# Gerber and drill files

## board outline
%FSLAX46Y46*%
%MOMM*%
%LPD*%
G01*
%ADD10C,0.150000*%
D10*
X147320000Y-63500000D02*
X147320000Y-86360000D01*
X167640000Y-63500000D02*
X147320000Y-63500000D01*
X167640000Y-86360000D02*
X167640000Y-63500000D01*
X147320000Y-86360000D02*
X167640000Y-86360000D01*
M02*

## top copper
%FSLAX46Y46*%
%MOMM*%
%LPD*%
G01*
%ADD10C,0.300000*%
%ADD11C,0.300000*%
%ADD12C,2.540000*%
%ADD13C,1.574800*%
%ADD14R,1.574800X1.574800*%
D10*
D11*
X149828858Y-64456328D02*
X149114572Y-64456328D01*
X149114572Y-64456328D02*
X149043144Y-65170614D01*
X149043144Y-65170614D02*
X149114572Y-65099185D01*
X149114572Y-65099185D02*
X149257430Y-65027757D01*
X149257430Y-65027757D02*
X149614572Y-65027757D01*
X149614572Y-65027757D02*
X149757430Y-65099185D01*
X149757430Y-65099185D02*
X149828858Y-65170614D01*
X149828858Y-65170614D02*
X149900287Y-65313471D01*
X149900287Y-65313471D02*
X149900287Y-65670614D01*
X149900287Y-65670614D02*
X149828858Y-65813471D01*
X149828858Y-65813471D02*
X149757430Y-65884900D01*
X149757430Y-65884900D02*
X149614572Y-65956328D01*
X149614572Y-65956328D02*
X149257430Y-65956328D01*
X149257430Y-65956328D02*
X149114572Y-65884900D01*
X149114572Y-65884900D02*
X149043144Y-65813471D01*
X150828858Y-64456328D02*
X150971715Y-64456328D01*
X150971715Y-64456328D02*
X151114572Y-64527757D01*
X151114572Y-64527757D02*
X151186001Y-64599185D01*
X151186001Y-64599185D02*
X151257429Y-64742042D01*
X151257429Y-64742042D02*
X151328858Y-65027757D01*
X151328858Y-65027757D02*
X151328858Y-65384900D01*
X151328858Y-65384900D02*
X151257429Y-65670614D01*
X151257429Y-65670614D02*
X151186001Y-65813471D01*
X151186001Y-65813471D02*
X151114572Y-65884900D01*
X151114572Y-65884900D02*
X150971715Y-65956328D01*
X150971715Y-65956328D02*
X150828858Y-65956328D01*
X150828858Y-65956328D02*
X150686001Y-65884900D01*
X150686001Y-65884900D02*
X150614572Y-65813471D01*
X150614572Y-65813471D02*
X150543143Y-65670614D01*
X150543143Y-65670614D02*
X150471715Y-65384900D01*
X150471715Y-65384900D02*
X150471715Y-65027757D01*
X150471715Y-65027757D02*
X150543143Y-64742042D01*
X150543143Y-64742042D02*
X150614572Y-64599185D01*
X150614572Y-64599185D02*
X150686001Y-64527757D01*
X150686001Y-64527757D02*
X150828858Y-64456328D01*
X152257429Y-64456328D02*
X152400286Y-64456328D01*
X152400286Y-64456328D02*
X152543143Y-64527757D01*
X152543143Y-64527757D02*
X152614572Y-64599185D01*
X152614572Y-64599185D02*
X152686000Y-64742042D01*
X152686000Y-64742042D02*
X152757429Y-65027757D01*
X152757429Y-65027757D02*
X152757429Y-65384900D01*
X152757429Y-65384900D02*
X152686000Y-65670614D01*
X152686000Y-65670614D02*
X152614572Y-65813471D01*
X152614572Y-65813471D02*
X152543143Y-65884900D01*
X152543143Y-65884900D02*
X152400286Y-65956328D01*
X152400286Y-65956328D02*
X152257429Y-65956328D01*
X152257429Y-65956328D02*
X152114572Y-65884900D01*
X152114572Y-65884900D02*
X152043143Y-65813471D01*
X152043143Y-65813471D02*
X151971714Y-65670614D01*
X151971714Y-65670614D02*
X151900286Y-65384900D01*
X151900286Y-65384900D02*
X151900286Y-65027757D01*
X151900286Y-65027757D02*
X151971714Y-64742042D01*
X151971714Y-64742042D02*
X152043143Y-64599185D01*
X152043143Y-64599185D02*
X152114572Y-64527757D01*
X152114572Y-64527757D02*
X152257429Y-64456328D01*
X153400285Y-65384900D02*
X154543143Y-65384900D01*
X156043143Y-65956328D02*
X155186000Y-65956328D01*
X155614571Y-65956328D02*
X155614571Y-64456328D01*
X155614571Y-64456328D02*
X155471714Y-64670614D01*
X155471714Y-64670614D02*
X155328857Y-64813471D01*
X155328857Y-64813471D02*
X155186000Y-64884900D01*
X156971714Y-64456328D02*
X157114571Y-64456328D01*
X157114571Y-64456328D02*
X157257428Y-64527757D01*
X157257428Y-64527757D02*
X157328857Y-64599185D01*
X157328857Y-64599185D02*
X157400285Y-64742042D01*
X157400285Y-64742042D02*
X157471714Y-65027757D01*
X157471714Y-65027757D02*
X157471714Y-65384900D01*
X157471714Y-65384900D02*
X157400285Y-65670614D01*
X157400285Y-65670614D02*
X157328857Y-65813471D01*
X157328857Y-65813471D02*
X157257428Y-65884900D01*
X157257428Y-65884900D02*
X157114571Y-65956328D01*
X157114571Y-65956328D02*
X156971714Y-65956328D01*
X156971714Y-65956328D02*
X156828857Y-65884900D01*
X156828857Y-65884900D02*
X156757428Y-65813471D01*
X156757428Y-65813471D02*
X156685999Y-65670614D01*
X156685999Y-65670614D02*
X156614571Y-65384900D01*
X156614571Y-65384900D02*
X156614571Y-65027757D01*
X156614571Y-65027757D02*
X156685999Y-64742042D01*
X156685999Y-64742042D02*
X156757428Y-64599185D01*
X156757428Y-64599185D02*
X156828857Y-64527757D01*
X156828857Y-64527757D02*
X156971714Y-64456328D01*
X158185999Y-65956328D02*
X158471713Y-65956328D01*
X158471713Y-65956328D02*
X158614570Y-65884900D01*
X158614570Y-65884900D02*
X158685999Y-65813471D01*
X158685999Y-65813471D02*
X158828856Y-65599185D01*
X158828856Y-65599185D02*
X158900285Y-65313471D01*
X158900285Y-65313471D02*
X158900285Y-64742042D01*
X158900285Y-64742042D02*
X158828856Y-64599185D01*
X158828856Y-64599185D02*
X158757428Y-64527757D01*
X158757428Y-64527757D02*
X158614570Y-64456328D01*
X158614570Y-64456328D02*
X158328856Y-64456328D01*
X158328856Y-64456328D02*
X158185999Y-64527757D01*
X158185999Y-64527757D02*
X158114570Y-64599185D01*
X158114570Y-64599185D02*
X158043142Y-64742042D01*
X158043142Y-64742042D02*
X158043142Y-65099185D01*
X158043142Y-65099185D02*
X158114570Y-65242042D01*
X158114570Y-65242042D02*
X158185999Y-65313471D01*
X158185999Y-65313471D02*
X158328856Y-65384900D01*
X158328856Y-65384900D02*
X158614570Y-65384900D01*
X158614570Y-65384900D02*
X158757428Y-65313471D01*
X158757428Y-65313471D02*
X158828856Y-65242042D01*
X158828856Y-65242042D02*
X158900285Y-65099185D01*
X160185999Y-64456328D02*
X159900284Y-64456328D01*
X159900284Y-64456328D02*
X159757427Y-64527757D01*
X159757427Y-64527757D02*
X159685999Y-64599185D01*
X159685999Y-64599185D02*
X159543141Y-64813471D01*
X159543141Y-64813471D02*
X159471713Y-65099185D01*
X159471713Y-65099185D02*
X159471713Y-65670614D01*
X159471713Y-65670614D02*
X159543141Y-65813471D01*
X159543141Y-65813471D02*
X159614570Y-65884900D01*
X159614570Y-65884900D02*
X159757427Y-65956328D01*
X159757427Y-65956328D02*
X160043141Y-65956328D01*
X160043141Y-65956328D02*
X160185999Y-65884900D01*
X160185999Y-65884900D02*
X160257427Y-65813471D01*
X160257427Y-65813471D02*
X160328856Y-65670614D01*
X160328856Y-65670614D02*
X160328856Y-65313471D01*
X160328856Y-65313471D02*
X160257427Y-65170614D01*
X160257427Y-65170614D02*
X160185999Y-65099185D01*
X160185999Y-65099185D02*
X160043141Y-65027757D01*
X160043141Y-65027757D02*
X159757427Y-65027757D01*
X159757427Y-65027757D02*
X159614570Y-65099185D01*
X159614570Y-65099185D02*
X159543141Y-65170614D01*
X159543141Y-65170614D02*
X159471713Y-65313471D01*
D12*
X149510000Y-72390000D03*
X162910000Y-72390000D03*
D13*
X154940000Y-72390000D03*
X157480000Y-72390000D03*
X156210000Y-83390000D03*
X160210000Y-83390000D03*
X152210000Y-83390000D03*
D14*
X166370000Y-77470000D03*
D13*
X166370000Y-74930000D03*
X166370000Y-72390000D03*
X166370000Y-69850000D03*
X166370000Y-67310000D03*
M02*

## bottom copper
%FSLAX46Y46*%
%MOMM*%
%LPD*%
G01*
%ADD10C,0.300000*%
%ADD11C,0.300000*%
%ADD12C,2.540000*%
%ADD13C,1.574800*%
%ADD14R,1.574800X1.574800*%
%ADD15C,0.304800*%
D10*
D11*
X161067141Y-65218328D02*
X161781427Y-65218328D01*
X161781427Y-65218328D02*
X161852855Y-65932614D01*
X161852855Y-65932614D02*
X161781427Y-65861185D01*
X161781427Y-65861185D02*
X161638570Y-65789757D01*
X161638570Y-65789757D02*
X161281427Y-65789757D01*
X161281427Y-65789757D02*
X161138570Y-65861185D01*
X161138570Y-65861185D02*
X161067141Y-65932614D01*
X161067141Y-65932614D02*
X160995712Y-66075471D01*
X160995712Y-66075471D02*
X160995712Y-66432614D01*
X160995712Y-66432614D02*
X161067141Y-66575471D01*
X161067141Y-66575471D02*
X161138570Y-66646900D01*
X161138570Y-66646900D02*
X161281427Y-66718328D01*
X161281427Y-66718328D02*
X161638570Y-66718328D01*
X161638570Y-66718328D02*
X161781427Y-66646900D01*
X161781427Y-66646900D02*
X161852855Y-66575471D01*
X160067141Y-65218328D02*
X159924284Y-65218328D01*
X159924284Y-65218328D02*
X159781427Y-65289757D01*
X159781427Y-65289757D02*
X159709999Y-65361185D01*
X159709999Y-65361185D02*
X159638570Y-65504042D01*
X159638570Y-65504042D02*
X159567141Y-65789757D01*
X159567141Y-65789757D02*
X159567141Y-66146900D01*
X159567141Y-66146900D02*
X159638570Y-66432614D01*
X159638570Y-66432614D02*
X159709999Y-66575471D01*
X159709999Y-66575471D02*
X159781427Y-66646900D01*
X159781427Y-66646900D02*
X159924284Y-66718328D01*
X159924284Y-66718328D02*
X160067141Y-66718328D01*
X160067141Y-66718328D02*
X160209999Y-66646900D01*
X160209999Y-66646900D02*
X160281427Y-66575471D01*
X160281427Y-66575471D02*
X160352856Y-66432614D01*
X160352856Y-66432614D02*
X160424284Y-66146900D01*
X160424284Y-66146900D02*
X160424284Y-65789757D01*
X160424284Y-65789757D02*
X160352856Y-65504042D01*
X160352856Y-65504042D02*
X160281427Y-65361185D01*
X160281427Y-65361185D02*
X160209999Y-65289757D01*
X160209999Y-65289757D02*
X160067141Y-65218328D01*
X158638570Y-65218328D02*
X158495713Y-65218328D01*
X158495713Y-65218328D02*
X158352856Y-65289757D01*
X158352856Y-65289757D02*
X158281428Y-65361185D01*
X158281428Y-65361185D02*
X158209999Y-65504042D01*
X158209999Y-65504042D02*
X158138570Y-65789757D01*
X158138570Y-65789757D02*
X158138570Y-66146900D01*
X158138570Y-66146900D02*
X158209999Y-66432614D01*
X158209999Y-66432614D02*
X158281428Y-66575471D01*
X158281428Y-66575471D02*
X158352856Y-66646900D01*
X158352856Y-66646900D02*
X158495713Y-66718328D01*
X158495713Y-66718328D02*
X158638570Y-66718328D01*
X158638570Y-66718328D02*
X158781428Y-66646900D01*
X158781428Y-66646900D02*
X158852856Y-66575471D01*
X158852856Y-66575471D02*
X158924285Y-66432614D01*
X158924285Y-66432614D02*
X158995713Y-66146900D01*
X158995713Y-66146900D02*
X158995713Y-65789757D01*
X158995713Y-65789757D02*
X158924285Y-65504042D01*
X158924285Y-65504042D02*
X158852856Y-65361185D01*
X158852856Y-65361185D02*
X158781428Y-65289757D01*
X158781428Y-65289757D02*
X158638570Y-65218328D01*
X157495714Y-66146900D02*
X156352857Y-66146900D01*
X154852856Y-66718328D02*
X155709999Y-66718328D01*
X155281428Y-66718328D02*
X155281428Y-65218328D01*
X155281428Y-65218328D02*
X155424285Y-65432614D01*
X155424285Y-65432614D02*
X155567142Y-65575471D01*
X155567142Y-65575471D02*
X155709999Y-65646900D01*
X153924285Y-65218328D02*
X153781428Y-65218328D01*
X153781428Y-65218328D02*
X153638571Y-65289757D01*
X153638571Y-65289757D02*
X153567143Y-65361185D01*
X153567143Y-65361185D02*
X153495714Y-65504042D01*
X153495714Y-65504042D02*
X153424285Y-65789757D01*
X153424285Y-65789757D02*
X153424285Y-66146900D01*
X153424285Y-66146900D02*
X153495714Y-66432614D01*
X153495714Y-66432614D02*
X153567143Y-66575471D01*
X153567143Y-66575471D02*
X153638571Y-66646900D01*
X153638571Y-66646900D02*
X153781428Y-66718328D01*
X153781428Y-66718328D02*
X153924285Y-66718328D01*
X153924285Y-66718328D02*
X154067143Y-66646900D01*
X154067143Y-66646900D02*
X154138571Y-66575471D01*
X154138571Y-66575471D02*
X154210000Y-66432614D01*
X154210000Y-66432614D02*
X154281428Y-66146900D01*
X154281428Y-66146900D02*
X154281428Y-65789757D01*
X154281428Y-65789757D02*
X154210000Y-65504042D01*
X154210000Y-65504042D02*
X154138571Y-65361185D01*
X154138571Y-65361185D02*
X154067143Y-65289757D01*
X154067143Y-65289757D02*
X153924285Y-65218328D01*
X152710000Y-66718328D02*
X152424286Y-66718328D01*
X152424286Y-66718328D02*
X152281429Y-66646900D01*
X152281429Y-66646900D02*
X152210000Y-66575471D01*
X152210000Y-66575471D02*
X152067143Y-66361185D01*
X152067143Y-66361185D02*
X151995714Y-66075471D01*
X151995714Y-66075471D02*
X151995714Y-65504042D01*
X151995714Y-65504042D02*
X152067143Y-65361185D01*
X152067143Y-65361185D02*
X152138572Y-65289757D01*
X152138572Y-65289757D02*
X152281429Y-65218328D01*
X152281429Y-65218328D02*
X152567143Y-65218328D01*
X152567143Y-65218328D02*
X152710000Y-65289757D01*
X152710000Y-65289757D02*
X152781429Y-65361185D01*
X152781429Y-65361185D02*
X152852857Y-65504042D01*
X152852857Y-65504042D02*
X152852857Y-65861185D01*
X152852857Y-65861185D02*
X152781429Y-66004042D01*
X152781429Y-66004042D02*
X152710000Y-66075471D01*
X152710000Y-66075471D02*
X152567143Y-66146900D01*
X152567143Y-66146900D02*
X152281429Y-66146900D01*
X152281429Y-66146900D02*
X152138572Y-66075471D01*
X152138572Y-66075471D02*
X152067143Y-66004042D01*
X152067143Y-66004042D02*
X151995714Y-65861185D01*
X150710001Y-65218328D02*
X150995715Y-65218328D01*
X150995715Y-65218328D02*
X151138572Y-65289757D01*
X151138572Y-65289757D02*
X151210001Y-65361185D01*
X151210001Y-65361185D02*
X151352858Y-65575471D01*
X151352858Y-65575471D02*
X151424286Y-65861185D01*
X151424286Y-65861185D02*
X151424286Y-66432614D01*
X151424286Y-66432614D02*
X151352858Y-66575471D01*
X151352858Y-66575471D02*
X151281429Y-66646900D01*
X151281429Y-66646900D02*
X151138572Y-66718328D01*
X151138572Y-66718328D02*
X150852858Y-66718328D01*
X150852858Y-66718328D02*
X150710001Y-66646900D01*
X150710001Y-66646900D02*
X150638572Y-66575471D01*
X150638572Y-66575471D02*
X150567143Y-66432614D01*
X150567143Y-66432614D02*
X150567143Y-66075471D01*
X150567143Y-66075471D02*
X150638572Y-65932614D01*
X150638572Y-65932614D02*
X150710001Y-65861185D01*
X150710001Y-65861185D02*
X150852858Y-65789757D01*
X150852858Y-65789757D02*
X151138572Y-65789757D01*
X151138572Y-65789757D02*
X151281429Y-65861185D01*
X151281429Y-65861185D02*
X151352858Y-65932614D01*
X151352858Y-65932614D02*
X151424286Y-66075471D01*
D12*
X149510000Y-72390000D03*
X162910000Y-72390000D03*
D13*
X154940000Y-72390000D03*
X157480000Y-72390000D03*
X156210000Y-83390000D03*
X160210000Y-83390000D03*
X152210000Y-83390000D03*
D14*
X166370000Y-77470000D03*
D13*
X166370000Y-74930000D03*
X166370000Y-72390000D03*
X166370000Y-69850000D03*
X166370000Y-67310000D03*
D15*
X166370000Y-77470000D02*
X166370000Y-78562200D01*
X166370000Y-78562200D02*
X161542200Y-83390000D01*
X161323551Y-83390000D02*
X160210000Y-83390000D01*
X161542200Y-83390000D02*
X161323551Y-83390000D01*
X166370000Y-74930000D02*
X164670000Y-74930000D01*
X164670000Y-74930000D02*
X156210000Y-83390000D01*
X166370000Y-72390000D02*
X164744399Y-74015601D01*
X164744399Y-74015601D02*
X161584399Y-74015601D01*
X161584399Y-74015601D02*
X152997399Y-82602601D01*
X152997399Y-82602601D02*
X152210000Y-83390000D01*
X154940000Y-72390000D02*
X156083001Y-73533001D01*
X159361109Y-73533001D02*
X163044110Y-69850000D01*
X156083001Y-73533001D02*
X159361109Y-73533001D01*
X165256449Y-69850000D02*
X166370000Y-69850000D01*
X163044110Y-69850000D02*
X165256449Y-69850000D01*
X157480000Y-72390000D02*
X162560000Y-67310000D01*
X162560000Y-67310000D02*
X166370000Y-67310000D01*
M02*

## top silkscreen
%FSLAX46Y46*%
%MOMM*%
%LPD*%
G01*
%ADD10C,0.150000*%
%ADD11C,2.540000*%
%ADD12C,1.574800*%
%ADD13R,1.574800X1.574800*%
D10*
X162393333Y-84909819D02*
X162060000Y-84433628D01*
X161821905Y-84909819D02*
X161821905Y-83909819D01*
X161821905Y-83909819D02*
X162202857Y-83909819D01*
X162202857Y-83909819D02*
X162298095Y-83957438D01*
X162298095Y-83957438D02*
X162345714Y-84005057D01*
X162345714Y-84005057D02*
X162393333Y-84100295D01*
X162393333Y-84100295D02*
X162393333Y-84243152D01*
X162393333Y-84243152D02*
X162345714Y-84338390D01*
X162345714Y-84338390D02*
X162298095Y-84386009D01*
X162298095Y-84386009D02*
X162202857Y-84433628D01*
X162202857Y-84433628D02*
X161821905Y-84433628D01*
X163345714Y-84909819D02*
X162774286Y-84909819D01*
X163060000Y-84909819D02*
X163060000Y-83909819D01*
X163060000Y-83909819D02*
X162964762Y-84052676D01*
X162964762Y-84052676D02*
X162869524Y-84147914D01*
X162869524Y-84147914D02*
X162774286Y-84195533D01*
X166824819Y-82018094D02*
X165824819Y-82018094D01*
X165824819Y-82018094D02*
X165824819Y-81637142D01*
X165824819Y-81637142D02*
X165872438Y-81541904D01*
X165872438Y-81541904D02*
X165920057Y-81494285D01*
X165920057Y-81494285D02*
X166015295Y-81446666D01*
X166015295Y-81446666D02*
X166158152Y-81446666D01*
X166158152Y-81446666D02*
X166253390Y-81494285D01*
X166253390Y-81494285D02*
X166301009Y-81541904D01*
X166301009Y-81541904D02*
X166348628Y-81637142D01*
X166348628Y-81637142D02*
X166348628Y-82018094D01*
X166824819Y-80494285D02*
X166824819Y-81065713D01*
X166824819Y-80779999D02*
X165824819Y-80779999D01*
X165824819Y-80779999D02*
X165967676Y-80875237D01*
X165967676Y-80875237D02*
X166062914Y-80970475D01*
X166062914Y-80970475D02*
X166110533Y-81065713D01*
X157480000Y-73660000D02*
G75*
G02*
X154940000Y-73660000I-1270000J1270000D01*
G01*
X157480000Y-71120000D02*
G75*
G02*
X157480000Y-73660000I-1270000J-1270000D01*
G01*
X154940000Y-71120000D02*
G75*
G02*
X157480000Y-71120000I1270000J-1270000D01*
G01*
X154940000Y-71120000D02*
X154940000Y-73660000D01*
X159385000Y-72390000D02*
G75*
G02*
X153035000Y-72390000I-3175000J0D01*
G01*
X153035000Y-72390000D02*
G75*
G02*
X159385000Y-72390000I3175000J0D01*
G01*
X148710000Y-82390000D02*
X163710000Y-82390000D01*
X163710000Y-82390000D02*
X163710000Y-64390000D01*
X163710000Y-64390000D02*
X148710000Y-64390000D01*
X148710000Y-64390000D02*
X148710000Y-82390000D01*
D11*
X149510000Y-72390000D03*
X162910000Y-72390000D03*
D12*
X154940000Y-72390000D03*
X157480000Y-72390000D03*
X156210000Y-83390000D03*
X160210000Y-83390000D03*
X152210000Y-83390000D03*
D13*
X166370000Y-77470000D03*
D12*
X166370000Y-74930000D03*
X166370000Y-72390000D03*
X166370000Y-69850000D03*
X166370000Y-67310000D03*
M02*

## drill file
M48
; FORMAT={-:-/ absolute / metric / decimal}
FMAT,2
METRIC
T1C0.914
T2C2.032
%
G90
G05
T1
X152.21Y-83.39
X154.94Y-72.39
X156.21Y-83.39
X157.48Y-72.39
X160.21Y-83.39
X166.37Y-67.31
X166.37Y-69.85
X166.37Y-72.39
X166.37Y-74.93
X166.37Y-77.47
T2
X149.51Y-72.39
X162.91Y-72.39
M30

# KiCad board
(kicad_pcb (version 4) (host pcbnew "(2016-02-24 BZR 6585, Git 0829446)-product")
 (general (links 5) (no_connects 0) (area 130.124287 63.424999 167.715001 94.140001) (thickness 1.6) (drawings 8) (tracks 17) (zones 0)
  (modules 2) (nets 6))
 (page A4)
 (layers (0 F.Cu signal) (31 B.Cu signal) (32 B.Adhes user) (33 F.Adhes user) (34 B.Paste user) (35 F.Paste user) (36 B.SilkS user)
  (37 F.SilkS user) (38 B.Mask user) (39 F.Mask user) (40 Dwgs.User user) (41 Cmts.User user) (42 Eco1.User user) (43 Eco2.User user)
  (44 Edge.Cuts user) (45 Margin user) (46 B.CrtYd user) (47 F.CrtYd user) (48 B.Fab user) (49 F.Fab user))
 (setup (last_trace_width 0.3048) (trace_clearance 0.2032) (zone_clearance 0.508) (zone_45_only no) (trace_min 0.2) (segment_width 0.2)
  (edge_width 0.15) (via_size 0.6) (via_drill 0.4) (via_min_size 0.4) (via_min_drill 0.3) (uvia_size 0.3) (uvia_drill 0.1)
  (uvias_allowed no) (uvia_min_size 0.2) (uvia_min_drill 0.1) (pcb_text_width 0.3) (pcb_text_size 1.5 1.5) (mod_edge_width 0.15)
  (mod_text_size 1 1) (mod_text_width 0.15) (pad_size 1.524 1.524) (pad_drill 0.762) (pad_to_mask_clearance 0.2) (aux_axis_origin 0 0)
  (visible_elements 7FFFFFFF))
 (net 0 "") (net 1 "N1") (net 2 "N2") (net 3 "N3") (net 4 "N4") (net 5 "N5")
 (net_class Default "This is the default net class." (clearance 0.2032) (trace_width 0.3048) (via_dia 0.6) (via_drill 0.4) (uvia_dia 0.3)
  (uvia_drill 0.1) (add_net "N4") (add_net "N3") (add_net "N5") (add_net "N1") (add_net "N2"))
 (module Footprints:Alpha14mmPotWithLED (layer F.Cu) (at 156.21 72.39)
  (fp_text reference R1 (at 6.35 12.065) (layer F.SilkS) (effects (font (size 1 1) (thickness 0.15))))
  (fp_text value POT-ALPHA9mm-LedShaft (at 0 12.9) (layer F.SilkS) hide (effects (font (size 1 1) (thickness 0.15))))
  (fp_arc (start 0 0) (end 1.27 1.27) (angle 90) (layer F.SilkS) (width 0.15))
  (fp_arc (start 0 0) (end 1.27 -1.27) (angle 90) (layer F.SilkS) (width 0.15))
  (fp_arc (start 0 0) (end -1.27 -1.27) (angle 90) (layer F.SilkS) (width 0.15))
  (fp_line (start -1.27 -1.27) (end -1.27 1.27) (layer F.SilkS) (width 0.15))
  (fp_circle (center 0 0) (end 3.175 0) (layer F.SilkS) (width 0.15))
  (fp_line (start -7.5 10) (end 7.5 10) (layer F.SilkS) (width 0.15))
  (fp_line (start 7.5 10) (end 7.5 -8) (layer F.SilkS) (width 0.15))
  (fp_line (start 7.5 -8) (end -7.5 -8) (layer F.SilkS) (width 0.15))
  (fp_line (start -7.5 -8) (end -7.5 10) (layer F.SilkS) (width 0.15))
  (pad "" thru_hole circle (at -6.7 0) (size 2.54 2.54) (drill 2.032) (layers *.Cu *.Mask F.SilkS))
  (pad "" thru_hole circle (at 6.7 0) (size 2.54 2.54) (drill 2.032) (layers *.Cu *.Mask F.SilkS))
  (pad 4 thru_hole circle (at -1.27 0) (size 1.5748 1.5748) (drill 0.9144) (layers *.Cu *.Mask F.SilkS) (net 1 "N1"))
  (pad 5 thru_hole circle (at 1.27 0) (size 1.5748 1.5748) (drill 0.9144) (layers *.Cu *.Mask F.SilkS) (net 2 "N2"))
  (pad 2 thru_hole circle (at 0 11) (size 1.5748 1.5748) (drill 0.9144) (layers *.Cu *.Mask F.SilkS) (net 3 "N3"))
  (pad 3 thru_hole circle (at 4 11) (size 1.5748 1.5748) (drill 0.9144) (layers *.Cu *.Mask F.SilkS) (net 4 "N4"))
  (pad 1 thru_hole circle (at -4 11) (size 1.5748 1.5748) (drill 0.9144) (layers *.Cu *.Mask F.SilkS) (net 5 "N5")))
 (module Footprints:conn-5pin (layer F.Cu) (at 166.37 72.39 90)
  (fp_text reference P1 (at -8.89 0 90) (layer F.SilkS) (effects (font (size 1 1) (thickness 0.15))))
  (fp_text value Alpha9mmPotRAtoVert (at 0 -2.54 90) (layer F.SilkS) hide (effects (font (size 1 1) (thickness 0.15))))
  (pad 1 thru_hole rect (at -5.08 0 90) (size 1.5748 1.5748) (drill 0.9144) (layers *.Cu *.Mask F.SilkS) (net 4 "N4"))
  (pad 2 thru_hole circle (at -2.54 0 90) (size 1.5748 1.5748) (drill 0.9144) (layers *.Cu *.Mask F.SilkS) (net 3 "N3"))
  (pad 3 thru_hole circle (at 0 0 90) (size 1.5748 1.5748) (drill 0.9144) (layers *.Cu *.Mask F.SilkS) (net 5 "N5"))
  (pad 4 thru_hole circle (at 2.54 0 90) (size 1.5748 1.5748) (drill 0.9144) (layers *.Cu *.Mask F.SilkS) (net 1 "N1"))
  (pad 5 thru_hole circle (at 5.08 0 90) (size 1.5748 1.5748) (drill 0.9144) (layers *.Cu *.Mask F.SilkS) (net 2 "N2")))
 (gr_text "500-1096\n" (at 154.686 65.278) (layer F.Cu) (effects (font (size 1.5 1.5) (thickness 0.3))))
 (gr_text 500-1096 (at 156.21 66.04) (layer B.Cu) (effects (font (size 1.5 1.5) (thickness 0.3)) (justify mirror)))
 (gr_line (start 147.32 63.5) (end 147.32 86.36) (layer Edge.Cuts) (width 0.15))
 (gr_line (start 167.64 63.5) (end 147.32 63.5) (layer Edge.Cuts) (width 0.15))
 (gr_line (start 167.64 86.36) (end 167.64 63.5) (layer Edge.Cuts) (width 0.15))
 (gr_line (start 147.32 86.36) (end 167.64 86.36) (layer Edge.Cuts) (width 0.15))
 (segment (start 166.37 77.47) (end 166.37 78.5622) (width 0.3048) (layer B.Cu) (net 4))
 (segment (start 166.37 78.5622) (end 161.5422 83.39) (width 0.3048) (layer B.Cu) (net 4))
 (segment (start 161.323551 83.39) (end 160.21 83.39) (width 0.3048) (layer B.Cu) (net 4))
 (segment (start 161.5422 83.39) (end 161.323551 83.39) (width 0.3048) (layer B.Cu) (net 4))
 (segment (start 166.37 74.93) (end 164.67 74.93) (width 0.3048) (layer B.Cu) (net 3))
 (segment (start 164.67 74.93) (end 156.21 83.39) (width 0.3048) (layer B.Cu) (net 3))
 (segment (start 166.37 72.39) (end 164.744399 74.015601) (width 0.3048) (layer B.Cu) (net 5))
 (segment (start 164.744399 74.015601) (end 161.584399 74.015601) (width 0.3048) (layer B.Cu) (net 5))
 (segment (start 161.584399 74.015601) (end 152.997399 82.602601) (width 0.3048) (layer B.Cu) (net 5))
 (segment (start 152.997399 82.602601) (end 152.21 83.39) (width 0.3048) (layer B.Cu) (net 5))
 (segment (start 154.94 72.39) (end 156.083001 73.533001) (width 0.3048) (layer B.Cu) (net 1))
 (segment (start 159.361109 73.533001) (end 163.04411 69.85) (width 0.3048) (layer B.Cu) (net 1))
 (segment (start 156.083001 73.533001) (end 159.361109 73.533001) (width 0.3048) (layer B.Cu) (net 1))
 (segment (start 165.256449 69.85) (end 166.37 69.85) (width 0.3048) (layer B.Cu) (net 1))
 (segment (start 163.04411 69.85) (end 165.256449 69.85) (width 0.3048) (layer B.Cu) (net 1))
 (segment (start 157.48 72.39) (end 162.56 67.31) (width 0.3048) (layer B.Cu) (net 2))
 (segment (start 162.56 67.31) (end 166.37 67.31) (width 0.3048) (layer B.Cu) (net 2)))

